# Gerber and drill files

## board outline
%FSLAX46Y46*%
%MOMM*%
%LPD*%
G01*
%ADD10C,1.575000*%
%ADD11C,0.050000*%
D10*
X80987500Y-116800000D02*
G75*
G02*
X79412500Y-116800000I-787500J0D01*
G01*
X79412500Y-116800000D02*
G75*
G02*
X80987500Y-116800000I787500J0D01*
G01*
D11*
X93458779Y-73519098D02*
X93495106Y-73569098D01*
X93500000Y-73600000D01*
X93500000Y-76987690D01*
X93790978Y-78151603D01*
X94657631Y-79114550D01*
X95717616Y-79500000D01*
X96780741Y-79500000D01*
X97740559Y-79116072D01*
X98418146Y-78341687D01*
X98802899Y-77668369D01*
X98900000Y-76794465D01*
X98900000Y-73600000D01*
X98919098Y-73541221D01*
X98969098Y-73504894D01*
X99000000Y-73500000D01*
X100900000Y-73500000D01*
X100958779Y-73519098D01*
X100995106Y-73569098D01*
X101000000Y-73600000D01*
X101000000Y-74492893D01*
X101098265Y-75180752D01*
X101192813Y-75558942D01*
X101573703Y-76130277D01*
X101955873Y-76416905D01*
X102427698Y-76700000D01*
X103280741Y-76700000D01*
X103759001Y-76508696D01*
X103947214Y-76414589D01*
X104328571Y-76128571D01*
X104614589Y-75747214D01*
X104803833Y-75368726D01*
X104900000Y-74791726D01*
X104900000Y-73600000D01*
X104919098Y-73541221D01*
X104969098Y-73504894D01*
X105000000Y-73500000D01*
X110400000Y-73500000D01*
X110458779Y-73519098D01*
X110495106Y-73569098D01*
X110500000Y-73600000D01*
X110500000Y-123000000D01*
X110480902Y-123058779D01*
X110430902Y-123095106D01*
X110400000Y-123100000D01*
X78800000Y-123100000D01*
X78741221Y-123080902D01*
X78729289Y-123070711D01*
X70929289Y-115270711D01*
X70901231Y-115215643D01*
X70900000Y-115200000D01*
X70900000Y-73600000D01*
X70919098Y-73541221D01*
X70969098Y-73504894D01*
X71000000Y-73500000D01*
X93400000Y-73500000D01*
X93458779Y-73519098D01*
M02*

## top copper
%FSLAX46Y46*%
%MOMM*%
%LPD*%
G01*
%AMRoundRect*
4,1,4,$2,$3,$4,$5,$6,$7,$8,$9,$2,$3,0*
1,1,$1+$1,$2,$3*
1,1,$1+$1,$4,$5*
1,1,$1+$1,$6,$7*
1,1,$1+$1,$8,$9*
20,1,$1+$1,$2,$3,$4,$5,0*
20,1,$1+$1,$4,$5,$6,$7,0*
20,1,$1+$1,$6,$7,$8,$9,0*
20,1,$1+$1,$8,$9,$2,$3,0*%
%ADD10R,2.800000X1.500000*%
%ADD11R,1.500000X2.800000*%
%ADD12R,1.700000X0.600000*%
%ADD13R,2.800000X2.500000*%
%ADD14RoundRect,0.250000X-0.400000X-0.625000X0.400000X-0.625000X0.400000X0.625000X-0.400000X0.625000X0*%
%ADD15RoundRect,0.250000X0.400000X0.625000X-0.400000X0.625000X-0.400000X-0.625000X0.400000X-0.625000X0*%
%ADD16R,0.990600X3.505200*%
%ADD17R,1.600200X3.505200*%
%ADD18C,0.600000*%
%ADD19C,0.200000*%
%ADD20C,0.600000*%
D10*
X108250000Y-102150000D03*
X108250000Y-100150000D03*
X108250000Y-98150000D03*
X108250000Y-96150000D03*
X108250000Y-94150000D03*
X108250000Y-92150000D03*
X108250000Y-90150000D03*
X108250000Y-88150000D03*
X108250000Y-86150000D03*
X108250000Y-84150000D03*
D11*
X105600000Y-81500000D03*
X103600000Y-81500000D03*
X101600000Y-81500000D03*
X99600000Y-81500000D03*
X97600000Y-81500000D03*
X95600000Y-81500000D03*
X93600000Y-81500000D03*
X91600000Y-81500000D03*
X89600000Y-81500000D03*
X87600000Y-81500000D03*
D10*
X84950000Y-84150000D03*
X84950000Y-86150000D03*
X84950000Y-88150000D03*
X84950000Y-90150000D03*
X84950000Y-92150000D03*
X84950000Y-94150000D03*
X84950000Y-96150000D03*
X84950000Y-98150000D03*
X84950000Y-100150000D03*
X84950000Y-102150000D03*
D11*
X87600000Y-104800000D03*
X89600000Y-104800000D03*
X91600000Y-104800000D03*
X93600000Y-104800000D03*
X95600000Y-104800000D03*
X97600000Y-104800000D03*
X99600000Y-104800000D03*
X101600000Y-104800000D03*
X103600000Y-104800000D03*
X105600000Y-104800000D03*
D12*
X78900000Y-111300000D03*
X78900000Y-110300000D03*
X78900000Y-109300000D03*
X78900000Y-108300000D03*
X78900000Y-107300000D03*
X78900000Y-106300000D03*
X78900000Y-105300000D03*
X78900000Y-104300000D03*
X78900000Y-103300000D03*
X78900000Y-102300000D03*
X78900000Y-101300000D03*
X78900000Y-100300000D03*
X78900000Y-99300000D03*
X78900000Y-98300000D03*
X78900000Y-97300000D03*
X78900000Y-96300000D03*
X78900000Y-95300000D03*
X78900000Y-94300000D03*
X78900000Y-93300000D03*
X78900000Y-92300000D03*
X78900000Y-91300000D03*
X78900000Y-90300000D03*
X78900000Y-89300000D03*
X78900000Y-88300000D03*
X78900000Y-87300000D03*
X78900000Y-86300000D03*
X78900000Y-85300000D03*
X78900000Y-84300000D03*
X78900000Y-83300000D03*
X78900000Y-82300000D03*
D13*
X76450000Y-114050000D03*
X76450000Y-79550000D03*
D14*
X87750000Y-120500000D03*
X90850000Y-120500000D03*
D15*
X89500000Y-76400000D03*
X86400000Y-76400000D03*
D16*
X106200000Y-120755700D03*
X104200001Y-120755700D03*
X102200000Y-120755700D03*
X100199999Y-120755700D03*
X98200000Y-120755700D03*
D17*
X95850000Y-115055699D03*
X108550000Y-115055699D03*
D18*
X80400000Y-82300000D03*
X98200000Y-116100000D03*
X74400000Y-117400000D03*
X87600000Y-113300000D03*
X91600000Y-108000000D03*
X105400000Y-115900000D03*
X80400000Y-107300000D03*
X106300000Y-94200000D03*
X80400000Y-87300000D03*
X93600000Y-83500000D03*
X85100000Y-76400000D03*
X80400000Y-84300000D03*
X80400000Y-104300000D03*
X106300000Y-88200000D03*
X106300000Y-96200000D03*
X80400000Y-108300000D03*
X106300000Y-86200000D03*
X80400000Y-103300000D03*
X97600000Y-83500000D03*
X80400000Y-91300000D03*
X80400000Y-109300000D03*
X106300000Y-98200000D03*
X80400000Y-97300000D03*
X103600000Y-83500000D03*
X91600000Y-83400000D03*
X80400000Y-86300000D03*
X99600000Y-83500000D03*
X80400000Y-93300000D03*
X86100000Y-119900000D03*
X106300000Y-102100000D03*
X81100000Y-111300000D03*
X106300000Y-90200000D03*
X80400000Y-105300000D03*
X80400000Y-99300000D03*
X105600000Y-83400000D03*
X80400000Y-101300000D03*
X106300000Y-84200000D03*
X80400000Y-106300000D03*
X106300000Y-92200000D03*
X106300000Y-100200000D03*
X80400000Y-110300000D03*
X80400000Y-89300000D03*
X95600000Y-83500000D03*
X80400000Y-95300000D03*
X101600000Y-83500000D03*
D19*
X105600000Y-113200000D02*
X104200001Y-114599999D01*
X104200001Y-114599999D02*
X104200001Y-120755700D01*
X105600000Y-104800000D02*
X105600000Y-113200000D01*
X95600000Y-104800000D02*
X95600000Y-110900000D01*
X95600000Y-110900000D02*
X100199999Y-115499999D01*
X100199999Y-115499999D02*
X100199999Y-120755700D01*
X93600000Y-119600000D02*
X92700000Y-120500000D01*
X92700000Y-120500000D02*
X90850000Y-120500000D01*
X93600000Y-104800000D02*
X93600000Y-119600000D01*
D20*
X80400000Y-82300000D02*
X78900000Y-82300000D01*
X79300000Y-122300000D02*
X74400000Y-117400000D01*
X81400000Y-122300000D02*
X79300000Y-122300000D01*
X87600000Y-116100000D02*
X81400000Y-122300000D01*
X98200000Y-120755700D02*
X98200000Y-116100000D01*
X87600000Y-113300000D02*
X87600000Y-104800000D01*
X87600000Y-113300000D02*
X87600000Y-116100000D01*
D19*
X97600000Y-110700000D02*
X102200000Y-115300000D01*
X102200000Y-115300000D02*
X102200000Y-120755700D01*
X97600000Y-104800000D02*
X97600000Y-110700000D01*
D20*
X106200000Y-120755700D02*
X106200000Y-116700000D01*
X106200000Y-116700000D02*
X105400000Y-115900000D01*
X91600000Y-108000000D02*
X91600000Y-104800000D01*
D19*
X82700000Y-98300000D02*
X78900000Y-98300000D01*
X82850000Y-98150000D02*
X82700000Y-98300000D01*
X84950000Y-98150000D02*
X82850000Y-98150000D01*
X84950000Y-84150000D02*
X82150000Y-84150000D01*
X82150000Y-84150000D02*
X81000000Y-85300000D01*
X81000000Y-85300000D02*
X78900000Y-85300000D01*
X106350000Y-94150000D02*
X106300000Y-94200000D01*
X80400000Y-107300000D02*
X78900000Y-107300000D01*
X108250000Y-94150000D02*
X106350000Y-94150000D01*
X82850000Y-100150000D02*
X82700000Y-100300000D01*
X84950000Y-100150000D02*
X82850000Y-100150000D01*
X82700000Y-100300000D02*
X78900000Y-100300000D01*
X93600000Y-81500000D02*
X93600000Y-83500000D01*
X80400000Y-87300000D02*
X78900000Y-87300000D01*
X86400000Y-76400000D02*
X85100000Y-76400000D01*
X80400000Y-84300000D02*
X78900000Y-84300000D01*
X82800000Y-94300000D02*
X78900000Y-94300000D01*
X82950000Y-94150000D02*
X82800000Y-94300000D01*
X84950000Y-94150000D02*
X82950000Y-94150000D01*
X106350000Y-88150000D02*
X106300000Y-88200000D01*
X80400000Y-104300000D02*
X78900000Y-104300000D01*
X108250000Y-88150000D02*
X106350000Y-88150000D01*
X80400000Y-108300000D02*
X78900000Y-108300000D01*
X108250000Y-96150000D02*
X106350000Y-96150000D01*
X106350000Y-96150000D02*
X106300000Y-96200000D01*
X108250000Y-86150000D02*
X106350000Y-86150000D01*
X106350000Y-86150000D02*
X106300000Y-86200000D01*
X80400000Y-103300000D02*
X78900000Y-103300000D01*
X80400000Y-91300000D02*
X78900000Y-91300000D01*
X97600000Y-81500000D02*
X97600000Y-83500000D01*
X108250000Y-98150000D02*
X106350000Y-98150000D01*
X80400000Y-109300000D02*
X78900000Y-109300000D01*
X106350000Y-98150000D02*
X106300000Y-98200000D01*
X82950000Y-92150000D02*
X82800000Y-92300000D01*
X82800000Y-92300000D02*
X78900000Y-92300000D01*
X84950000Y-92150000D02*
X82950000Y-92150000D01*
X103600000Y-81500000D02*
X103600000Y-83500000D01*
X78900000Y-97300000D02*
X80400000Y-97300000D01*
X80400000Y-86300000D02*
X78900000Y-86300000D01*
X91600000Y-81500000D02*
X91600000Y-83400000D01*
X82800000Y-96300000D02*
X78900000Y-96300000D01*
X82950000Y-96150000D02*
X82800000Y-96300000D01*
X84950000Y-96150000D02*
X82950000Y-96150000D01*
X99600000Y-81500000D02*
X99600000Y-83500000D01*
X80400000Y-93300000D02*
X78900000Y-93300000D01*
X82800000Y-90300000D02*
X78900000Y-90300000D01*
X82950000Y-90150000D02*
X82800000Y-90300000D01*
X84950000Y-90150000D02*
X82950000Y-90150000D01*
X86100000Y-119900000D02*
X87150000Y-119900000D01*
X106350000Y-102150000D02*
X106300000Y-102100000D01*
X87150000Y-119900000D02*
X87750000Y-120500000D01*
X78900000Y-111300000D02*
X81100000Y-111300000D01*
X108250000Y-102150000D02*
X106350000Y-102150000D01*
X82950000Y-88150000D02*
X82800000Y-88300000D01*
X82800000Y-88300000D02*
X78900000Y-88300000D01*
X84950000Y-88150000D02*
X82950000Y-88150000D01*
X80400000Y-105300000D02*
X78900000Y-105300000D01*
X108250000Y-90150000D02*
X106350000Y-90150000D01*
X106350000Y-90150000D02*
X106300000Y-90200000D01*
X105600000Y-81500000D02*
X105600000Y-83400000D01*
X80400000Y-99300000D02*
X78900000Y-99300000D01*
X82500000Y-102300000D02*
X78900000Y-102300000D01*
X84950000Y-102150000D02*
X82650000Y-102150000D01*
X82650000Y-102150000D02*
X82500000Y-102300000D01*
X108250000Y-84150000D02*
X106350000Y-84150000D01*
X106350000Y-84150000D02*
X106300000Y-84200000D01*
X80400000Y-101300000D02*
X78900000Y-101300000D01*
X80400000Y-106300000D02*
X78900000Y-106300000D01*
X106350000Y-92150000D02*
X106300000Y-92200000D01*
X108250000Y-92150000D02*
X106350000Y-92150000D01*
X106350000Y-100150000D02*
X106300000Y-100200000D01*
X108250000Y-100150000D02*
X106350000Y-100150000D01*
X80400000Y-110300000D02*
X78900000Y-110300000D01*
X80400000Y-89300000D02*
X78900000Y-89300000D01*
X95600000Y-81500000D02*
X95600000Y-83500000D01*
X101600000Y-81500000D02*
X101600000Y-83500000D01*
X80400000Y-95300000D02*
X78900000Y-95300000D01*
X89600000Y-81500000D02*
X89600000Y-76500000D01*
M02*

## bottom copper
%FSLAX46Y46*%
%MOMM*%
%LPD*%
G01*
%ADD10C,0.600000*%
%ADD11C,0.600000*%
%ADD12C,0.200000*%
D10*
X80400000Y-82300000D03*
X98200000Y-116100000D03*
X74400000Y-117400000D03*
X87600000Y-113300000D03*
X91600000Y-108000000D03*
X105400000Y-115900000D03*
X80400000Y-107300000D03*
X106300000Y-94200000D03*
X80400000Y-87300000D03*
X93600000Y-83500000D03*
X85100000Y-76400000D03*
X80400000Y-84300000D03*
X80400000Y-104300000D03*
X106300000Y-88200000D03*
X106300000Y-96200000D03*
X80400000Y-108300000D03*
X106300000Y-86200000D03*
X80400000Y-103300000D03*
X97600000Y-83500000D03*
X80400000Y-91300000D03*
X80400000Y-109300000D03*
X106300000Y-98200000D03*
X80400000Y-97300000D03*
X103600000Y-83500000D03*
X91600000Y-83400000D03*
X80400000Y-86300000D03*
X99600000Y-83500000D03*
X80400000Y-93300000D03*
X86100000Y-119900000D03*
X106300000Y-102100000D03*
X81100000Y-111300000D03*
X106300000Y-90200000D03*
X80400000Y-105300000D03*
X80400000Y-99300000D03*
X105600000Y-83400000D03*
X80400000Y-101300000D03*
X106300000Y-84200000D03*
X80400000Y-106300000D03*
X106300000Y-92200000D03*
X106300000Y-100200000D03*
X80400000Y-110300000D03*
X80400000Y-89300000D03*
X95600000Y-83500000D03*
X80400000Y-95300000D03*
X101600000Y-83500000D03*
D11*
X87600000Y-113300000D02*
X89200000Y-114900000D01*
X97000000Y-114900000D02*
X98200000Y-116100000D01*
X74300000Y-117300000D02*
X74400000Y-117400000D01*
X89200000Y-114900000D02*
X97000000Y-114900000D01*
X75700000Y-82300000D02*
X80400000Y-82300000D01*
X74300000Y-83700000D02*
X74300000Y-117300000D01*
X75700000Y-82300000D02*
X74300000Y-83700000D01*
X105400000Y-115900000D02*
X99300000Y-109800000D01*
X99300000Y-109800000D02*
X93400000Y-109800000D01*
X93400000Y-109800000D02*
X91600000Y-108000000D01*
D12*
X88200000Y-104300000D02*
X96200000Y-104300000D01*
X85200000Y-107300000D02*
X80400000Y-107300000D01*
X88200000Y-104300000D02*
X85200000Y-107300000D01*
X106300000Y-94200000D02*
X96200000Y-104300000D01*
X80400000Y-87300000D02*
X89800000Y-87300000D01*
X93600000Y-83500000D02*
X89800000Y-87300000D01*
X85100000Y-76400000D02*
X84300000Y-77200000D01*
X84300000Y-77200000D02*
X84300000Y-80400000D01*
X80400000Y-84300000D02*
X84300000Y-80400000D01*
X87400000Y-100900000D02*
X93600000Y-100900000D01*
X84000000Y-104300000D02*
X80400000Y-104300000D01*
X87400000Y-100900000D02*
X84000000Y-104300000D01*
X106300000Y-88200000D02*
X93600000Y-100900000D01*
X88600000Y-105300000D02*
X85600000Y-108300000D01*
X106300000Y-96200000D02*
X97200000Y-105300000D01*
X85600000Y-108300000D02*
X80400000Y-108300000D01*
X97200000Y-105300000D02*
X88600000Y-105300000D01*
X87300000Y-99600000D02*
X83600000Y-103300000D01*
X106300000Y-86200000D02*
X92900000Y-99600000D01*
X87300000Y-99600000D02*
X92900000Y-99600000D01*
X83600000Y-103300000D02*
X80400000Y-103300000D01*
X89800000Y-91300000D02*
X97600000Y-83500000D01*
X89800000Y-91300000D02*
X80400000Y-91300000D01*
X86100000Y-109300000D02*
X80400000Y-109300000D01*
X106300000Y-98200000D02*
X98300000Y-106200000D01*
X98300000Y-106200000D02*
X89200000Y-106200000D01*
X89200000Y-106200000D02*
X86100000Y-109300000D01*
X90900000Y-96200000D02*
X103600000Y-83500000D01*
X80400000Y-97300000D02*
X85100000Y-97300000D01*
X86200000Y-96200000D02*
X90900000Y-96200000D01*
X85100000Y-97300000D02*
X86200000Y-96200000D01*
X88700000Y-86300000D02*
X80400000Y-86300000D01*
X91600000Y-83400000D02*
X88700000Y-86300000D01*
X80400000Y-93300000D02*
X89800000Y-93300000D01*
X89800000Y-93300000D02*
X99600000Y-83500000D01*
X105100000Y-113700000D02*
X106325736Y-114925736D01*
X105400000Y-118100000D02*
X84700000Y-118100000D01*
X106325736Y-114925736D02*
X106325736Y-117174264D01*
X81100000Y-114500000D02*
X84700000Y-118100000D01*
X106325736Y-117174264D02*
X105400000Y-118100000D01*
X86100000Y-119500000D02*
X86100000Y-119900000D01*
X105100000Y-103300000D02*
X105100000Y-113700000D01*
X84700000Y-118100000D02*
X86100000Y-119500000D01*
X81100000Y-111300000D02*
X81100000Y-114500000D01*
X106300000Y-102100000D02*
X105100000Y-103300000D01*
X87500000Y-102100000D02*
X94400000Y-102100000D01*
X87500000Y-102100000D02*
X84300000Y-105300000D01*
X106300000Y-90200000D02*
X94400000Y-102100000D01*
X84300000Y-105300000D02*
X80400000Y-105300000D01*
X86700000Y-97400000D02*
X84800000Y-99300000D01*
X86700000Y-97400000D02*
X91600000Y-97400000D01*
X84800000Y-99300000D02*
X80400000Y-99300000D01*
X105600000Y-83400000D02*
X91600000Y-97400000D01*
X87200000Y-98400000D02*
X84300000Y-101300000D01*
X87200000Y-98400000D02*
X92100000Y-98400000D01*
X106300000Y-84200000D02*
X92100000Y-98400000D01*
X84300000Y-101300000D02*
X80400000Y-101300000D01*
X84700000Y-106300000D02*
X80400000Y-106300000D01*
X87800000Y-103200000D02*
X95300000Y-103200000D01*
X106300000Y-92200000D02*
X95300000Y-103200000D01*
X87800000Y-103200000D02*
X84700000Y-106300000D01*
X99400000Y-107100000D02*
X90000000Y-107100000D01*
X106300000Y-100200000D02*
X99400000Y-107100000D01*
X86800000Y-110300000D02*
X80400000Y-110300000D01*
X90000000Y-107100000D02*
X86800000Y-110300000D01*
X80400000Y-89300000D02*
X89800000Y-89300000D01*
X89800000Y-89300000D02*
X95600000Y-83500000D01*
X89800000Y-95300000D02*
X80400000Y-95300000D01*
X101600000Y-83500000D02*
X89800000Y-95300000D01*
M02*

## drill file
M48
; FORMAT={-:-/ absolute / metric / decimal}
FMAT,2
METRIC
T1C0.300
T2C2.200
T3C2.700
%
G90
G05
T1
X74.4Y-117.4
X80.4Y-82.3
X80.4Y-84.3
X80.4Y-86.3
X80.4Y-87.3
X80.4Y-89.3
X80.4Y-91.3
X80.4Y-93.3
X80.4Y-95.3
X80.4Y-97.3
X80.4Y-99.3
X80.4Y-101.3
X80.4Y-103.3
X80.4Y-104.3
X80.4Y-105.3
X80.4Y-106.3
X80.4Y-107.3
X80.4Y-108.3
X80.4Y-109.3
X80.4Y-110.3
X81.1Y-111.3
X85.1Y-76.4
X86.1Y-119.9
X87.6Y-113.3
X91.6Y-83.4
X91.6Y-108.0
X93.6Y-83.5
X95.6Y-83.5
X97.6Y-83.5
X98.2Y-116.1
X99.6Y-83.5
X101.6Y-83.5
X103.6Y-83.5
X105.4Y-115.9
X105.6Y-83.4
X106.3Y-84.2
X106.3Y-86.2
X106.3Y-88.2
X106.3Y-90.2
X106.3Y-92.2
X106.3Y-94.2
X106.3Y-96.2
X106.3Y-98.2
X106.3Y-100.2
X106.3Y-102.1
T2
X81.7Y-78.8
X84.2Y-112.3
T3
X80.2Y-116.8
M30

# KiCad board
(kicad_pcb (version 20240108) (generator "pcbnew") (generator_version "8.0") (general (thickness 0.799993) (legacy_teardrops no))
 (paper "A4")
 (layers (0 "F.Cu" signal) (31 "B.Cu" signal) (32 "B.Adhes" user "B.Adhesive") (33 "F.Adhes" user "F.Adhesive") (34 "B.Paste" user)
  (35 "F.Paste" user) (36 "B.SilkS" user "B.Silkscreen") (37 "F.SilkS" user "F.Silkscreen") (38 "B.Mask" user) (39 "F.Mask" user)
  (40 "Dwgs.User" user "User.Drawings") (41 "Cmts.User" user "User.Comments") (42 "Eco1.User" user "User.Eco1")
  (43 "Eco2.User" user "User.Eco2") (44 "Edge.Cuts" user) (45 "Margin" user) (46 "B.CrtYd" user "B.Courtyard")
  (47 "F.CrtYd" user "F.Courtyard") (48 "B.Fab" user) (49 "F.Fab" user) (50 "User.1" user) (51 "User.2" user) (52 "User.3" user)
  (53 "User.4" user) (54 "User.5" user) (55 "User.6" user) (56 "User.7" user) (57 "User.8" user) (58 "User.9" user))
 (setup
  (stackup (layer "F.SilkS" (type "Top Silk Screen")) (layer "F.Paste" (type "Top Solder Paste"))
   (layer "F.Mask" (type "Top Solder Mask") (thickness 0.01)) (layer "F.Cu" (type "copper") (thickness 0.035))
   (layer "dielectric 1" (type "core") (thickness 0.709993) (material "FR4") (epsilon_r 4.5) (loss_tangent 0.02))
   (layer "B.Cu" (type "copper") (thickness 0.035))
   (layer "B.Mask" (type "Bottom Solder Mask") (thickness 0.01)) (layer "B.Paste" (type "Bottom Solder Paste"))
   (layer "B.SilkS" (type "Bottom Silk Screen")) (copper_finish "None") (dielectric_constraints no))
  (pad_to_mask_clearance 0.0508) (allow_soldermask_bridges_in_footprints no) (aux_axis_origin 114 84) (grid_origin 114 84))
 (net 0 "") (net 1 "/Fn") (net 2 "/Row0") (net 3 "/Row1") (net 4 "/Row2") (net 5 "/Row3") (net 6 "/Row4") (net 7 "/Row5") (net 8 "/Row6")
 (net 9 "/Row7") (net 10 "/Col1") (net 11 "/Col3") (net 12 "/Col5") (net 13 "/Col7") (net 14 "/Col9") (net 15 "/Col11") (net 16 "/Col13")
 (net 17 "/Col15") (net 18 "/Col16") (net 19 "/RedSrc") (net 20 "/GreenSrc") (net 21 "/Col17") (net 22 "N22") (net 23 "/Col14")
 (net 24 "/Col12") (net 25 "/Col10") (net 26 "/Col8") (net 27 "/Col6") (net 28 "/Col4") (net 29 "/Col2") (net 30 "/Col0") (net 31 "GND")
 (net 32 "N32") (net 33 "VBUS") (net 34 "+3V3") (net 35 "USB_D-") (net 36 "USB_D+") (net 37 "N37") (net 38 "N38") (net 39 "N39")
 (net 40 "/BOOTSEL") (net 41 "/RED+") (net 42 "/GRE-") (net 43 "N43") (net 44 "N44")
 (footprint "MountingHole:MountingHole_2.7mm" (layer "F.Cu") (at 80.2 116.8)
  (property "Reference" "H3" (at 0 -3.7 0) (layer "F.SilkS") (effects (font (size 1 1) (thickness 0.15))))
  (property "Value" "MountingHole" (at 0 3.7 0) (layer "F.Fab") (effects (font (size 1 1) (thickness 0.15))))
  (pad "" np_thru_hole circle (at 0 0) (size 2.7 2.7) (drill 2.7) (layers "*.Cu" "*.Mask")))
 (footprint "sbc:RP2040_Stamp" (layer "F.Cu") (at 96.6 93.15 180)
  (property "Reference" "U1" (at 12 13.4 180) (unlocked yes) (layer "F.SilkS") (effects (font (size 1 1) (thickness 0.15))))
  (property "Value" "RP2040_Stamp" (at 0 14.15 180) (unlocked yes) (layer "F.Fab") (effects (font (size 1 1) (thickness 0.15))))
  (pad "1" smd rect (at -11.65 -9 180) (size 2.8 1.5) (layers "F.Cu" "F.Paste" "F.Mask") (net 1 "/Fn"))
  (pad "2" smd rect (at -11.65 -7 180) (size 2.8 1.5) (layers "F.Cu" "F.Paste" "F.Mask") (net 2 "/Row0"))
  (pad "3" smd rect (at -11.65 -5 180) (size 2.8 1.5) (layers "F.Cu" "F.Paste" "F.Mask") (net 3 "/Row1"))
  (pad "4" smd rect (at -11.65 -3 180) (size 2.8 1.5) (layers "F.Cu" "F.Paste" "F.Mask") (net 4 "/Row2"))
  (pad "5" smd rect (at -11.65 -1 180) (size 2.8 1.5) (layers "F.Cu" "F.Paste" "F.Mask") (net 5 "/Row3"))
  (pad "6" smd rect (at -11.65 1 180) (size 2.8 1.5) (layers "F.Cu" "F.Paste" "F.Mask") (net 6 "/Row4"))
  (pad "7" smd rect (at -11.65 3 180) (size 2.8 1.5) (layers "F.Cu" "F.Paste" "F.Mask") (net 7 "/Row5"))
  (pad "8" smd rect (at -11.65 5 180) (size 2.8 1.5) (layers "F.Cu" "F.Paste" "F.Mask") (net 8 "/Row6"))
  (pad "9" smd rect (at -11.65 7 180) (size 2.8 1.5) (layers "F.Cu" "F.Paste" "F.Mask") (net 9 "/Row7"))
  (pad "10" smd rect (at -11.65 9 180) (size 2.8 1.5) (layers "F.Cu" "F.Paste" "F.Mask") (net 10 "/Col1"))
  (pad "11" smd rect (at -9 11.65 90) (size 2.8 1.5) (layers "F.Cu" "F.Paste" "F.Mask") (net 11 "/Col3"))
  (pad "12" smd rect (at -7 11.65 90) (size 2.8 1.5) (layers "F.Cu" "F.Paste" "F.Mask") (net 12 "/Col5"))
  (pad "13" smd rect (at -5 11.65 90) (size 2.8 1.5) (layers "F.Cu" "F.Paste" "F.Mask") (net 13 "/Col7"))
  (pad "14" smd rect (at -3 11.65 90) (size 2.8 1.5) (layers "F.Cu" "F.Paste" "F.Mask") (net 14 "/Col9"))
  (pad "15" smd rect (at -1 11.65 90) (size 2.8 1.5) (layers "F.Cu" "F.Paste" "F.Mask") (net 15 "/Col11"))
  (pad "16" smd rect (at 1 11.65 90) (size 2.8 1.5) (layers "F.Cu" "F.Paste" "F.Mask") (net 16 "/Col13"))
  (pad "17" smd rect (at 3 11.65 90) (size 2.8 1.5) (layers "F.Cu" "F.Paste" "F.Mask") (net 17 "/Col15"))
  (pad "18" smd rect (at 5 11.65 90) (size 2.8 1.5) (layers "F.Cu" "F.Paste" "F.Mask") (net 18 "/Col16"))
  (pad "19" smd rect (at 7 11.65 90) (size 2.8 1.5) (layers "F.Cu" "F.Paste" "F.Mask") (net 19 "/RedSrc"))
  (pad "20" smd rect (at 9 11.65 90) (size 2.8 1.5) (layers "F.Cu" "F.Paste" "F.Mask") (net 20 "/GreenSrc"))
  (pad "21" smd rect (at 11.65 9 180) (size 2.8 1.5) (layers "F.Cu" "F.Paste" "F.Mask") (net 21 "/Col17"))
  (pad "22" smd rect (at 11.65 7 180) (size 2.8 1.5) (layers "F.Cu" "F.Paste" "F.Mask") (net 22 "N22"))
  (pad "23" smd rect (at 11.65 5 180) (size 2.8 1.5) (layers "F.Cu" "F.Paste" "F.Mask") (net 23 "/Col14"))
  (pad "24" smd rect (at 11.65 3 180) (size 2.8 1.5) (layers "F.Cu" "F.Paste" "F.Mask") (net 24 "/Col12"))
  (pad "25" smd rect (at 11.65 1 180) (size 2.8 1.5) (layers "F.Cu" "F.Paste" "F.Mask") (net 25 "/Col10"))
  (pad "26" smd rect (at 11.65 -1 180) (size 2.8 1.5) (layers "F.Cu" "F.Paste" "F.Mask") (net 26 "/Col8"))
  (pad "27" smd rect (at 11.65 -3 180) (size 2.8 1.5) (layers "F.Cu" "F.Paste" "F.Mask") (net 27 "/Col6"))
  (pad "28" smd rect (at 11.65 -5 180) (size 2.8 1.5) (layers "F.Cu" "F.Paste" "F.Mask") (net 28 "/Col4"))
  (pad "29" smd rect (at 11.65 -7 180) (size 2.8 1.5) (layers "F.Cu" "F.Paste" "F.Mask") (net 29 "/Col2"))
  (pad "30" smd rect (at 11.65 -9 180) (size 2.8 1.5) (layers "F.Cu" "F.Paste" "F.Mask") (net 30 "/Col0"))
  (pad "31" smd rect (at 9 -11.65 90) (size 2.8 1.5) (layers "F.Cu" "F.Paste" "F.Mask") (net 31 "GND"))
  (pad "32" smd rect (at 7 -11.65 90) (size 2.8 1.5) (layers "F.Cu" "F.Paste" "F.Mask") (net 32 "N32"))
  (pad "33" smd rect (at 5 -11.65 90) (size 2.8 1.5) (layers "F.Cu" "F.Paste" "F.Mask") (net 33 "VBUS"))
  (pad "34" smd rect (at 3 -11.65 90) (size 2.8 1.5) (layers "F.Cu" "F.Paste" "F.Mask") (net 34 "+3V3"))
  (pad "35" smd rect (at 1 -11.65 90) (size 2.8 1.5) (layers "F.Cu" "F.Paste" "F.Mask") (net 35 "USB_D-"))
  (pad "36" smd rect (at -1 -11.65 90) (size 2.8 1.5) (layers "F.Cu" "F.Paste" "F.Mask") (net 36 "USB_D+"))
  (pad "37" smd rect (at -3 -11.65 90) (size 2.8 1.5) (layers "F.Cu" "F.Paste" "F.Mask") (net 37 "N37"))
  (pad "38" smd rect (at -5 -11.65 90) (size 2.8 1.5) (layers "F.Cu" "F.Paste" "F.Mask") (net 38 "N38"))
  (pad "39" smd rect (at -7 -11.65 90) (size 2.8 1.5) (layers "F.Cu" "F.Paste" "F.Mask") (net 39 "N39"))
  (pad "40" smd rect (at -9 -11.65 90) (size 2.8 1.5) (layers "F.Cu" "F.Paste" "F.Mask") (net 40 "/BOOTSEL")))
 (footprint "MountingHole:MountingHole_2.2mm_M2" (layer "F.Cu") (at 81.7 78.8)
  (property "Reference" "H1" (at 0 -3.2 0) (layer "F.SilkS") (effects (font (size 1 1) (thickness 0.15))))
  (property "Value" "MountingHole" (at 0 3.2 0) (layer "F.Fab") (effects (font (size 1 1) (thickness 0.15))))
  (pad "" np_thru_hole circle (at 0 0) (size 2.2 2.2) (drill 2.2) (layers "*.Cu" "*.Mask")))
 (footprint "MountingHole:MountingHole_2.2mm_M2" (layer "F.Cu") (at 84.2 112.3)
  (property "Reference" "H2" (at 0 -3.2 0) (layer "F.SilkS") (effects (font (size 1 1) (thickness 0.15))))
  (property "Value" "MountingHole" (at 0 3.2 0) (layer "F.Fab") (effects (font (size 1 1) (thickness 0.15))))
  (pad "" np_thru_hole circle (at 0 0) (size 2.2 2.2) (drill 2.2) (layers "*.Cu" "*.Mask")))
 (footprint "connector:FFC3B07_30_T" (layer "F.Cu") (at 76.45 96.8 -90)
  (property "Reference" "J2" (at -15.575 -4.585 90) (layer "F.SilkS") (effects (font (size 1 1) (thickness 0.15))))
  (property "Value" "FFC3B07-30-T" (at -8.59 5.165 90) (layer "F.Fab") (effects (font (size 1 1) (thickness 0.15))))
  (pad "1" smd rect (at 14.5 -2.45 270) (size 0.6 1.7) (layers "F.Cu" "F.Paste" "F.Mask") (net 1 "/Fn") (solder_mask_margin 0.102))
  (pad "2" smd rect (at 13.5 -2.45 270) (size 0.6 1.7) (layers "F.Cu" "F.Paste" "F.Mask") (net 2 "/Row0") (solder_mask_margin 0.102))
  (pad "3" smd rect (at 12.5 -2.45 270) (size 0.6 1.7) (layers "F.Cu" "F.Paste" "F.Mask") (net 3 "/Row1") (solder_mask_margin 0.102))
  (pad "4" smd rect (at 11.5 -2.45 270) (size 0.6 1.7) (layers "F.Cu" "F.Paste" "F.Mask") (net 4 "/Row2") (solder_mask_margin 0.102))
  (pad "5" smd rect (at 10.5 -2.45 270) (size 0.6 1.7) (layers "F.Cu" "F.Paste" "F.Mask") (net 5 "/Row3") (solder_mask_margin 0.102))
  (pad "6" smd rect (at 9.5 -2.45 270) (size 0.6 1.7) (layers "F.Cu" "F.Paste" "F.Mask") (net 6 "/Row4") (solder_mask_margin 0.102))
  (pad "7" smd rect (at 8.5 -2.45 270) (size 0.6 1.7) (layers "F.Cu" "F.Paste" "F.Mask") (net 7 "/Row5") (solder_mask_margin 0.102))
  (pad "8" smd rect (at 7.5 -2.45 270) (size 0.6 1.7) (layers "F.Cu" "F.Paste" "F.Mask") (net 8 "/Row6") (solder_mask_margin 0.102))
  (pad "9" smd rect (at 6.5 -2.45 270) (size 0.6 1.7) (layers "F.Cu" "F.Paste" "F.Mask") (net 9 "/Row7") (solder_mask_margin 0.102))
  (pad "10" smd rect (at 5.5 -2.45 270) (size 0.6 1.7) (layers "F.Cu" "F.Paste" "F.Mask") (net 30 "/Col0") (solder_mask_margin 0.102))
  (pad "11" smd rect (at 4.5 -2.45 270) (size 0.6 1.7) (layers "F.Cu" "F.Paste" "F.Mask") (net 10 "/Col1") (solder_mask_margin 0.102))
  (pad "12" smd rect (at 3.5 -2.45 270) (size 0.6 1.7) (layers "F.Cu" "F.Paste" "F.Mask") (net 29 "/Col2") (solder_mask_margin 0.102))
  (pad "13" smd rect (at 2.5 -2.45 270) (size 0.6 1.7) (layers "F.Cu" "F.Paste" "F.Mask") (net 11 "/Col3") (solder_mask_margin 0.102))
  (pad "14" smd rect (at 1.5 -2.45 270) (size 0.6 1.7) (layers "F.Cu" "F.Paste" "F.Mask") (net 28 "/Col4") (solder_mask_margin 0.102))
  (pad "15" smd rect (at 0.5 -2.45 270) (size 0.6 1.7) (layers "F.Cu" "F.Paste" "F.Mask") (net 12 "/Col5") (solder_mask_margin 0.102))
  (pad "16" smd rect (at -0.5 -2.45 270) (size 0.6 1.7) (layers "F.Cu" "F.Paste" "F.Mask") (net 27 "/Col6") (solder_mask_margin 0.102))
  (pad "17" smd rect (at -1.5 -2.45 270) (size 0.6 1.7) (layers "F.Cu" "F.Paste" "F.Mask") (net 13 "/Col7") (solder_mask_margin 0.102))
  (pad "18" smd rect (at -2.5 -2.45 270) (size 0.6 1.7) (layers "F.Cu" "F.Paste" "F.Mask") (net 26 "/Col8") (solder_mask_margin 0.102))
  (pad "19" smd rect (at -3.5 -2.45 270) (size 0.6 1.7) (layers "F.Cu" "F.Paste" "F.Mask") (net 14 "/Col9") (solder_mask_margin 0.102))
  (pad "20" smd rect (at -4.5 -2.45 270) (size 0.6 1.7) (layers "F.Cu" "F.Paste" "F.Mask") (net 25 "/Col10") (solder_mask_margin 0.102))
  (pad "21" smd rect (at -5.5 -2.45 270) (size 0.6 1.7) (layers "F.Cu" "F.Paste" "F.Mask") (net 15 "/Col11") (solder_mask_margin 0.102))
  (pad "22" smd rect (at -6.5 -2.45 270) (size 0.6 1.7) (layers "F.Cu" "F.Paste" "F.Mask") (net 24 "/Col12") (solder_mask_margin 0.102))
  (pad "23" smd rect (at -7.5 -2.45 270) (size 0.6 1.7) (layers "F.Cu" "F.Paste" "F.Mask") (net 16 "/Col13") (solder_mask_margin 0.102))
  (pad "24" smd rect (at -8.5 -2.45 270) (size 0.6 1.7) (layers "F.Cu" "F.Paste" "F.Mask") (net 23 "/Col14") (solder_mask_margin 0.102))
  (pad "25" smd rect (at -9.5 -2.45 270) (size 0.6 1.7) (layers "F.Cu" "F.Paste" "F.Mask") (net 17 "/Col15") (solder_mask_margin 0.102))
  (pad "26" smd rect (at -10.5 -2.45 270) (size 0.6 1.7) (layers "F.Cu" "F.Paste" "F.Mask") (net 18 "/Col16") (solder_mask_margin 0.102))
  (pad "27" smd rect (at -11.5 -2.45 270) (size 0.6 1.7) (layers "F.Cu" "F.Paste" "F.Mask") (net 21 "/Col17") (solder_mask_margin 0.102))
  (pad "28" smd rect (at -12.5 -2.45 270) (size 0.6 1.7) (layers "F.Cu" "F.Paste" "F.Mask") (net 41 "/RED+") (solder_mask_margin 0.102))
  (pad "29" smd rect (at -13.5 -2.45 270) (size 0.6 1.7) (layers "F.Cu" "F.Paste" "F.Mask") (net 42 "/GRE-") (solder_mask_margin 0.102))
  (pad "30" smd rect (at -14.5 -2.45 270) (size 0.6 1.7) (layers "F.Cu" "F.Paste" "F.Mask") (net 31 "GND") (solder_mask_margin 0.102))
  (pad "S1" smd rect (at 17.25 0 270) (size 2.5 2.8) (layers "F.Cu" "F.Paste" "F.Mask") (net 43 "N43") (solder_mask_margin 0.102))
  (pad "S2" smd rect (at -17.25 0 270) (size 2.5 2.8) (layers "F.Cu" "F.Paste" "F.Mask") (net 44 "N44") (solder_mask_margin 0.102)))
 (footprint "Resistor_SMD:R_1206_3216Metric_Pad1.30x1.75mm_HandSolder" (layer "F.Cu") (at 89.3 120.5)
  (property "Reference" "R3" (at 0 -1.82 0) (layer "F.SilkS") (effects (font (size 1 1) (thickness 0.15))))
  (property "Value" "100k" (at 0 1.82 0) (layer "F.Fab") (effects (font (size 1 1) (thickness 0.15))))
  (pad "1" smd roundrect (at -1.55 0) (size 1.3 1.75) (layers "F.Cu" "F.Paste" "F.Mask") (roundrect_rratio 0.192308) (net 1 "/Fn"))
  (pad "2" smd roundrect (at 1.55 0) (size 1.3 1.75) (layers "F.Cu" "F.Paste" "F.Mask") (roundrect_rratio 0.192308) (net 34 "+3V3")))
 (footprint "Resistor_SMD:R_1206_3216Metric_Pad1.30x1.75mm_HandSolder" (layer "F.Cu") (at 87.95 76.4 180)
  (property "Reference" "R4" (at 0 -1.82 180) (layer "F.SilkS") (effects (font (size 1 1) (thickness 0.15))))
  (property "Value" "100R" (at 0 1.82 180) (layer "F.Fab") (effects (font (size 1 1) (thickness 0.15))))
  (pad "1" smd roundrect (at -1.55 0 180) (size 1.3 1.75) (layers "F.Cu" "F.Paste" "F.Mask") (roundrect_rratio 0.192308) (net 19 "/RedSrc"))
  (pad "2" smd roundrect (at 1.55 0 180) (size 1.3 1.75) (layers "F.Cu" "F.Paste" "F.Mask") (roundrect_rratio 0.192308) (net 41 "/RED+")))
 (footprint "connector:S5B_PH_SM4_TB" (layer "F.Cu") (at 102.2 117.3)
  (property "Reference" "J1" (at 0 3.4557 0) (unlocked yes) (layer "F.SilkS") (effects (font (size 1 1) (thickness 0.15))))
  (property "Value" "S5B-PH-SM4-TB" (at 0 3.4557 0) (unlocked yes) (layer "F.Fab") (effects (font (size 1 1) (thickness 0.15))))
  (pad "1" smd rect (at 4 3.4557) (size 0.9906 3.5052) (layers "F.Cu" "F.Paste" "F.Mask") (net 33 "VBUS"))
  (pad "2" smd rect (at 2.000001 3.4557) (size 0.9906 3.5052) (layers "F.Cu" "F.Paste" "F.Mask") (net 40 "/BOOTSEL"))
  (pad "3" smd rect (at 0 3.4557) (size 0.9906 3.5052) (layers "F.Cu" "F.Paste" "F.Mask") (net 36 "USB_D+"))
  (pad "4" smd rect (at -2.000001 3.4557) (size 0.9906 3.5052) (layers "F.Cu" "F.Paste" "F.Mask") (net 35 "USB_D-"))
  (pad "5" smd rect (at -4 3.4557) (size 0.9906 3.5052) (layers "F.Cu" "F.Paste" "F.Mask") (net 31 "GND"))
  (pad "6" smd rect (at -6.35 -2.244301) (size 1.6002 3.5052) (layers "F.Cu" "F.Paste" "F.Mask"))
  (pad "7" smd rect (at 6.35 -2.244301) (size 1.6002 3.5052) (layers "F.Cu" "F.Paste" "F.Mask")))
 (gr_circle (center 80.2 116.8) (end 81.75 116.8) (stroke (width 0.05) (type solid)) (fill solid) (layer "Edge.Cuts"))
 (gr_poly
  (pts (xy 93.458779 73.519098) (xy 93.495106 73.569098) (xy 93.5 73.6) (xy 93.5 76.98769) (xy 93.790978 78.151603) (xy 94.657631 79.11455)
   (xy 95.717616 79.5) (xy 96.780741 79.5) (xy 97.740559 79.116072) (xy 98.418146 78.341687) (xy 98.802899 77.668369) (xy 98.9 76.794465)
   (xy 98.9 73.6) (xy 98.919098 73.541221) (xy 98.969098 73.504894) (xy 99 73.5) (xy 100.9 73.5) (xy 100.958779 73.519098)
   (xy 100.995106 73.569098) (xy 101 73.6) (xy 101 74.492893) (xy 101.098265 75.180752) (xy 101.192813 75.558942) (xy 101.573703 76.130277)
   (xy 101.955873 76.416905) (xy 102.427698 76.7) (xy 103.280741 76.7) (xy 103.759001 76.508696) (xy 103.947214 76.414589)
   (xy 104.328571 76.128571) (xy 104.614589 75.747214) (xy 104.803833 75.368726) (xy 104.9 74.791726) (xy 104.9 73.6)
   (xy 104.919098 73.541221) (xy 104.969098 73.504894) (xy 105 73.5) (xy 110.4 73.5) (xy 110.458779 73.519098) (xy 110.495106 73.569098)
   (xy 110.5 73.6) (xy 110.5 123) (xy 110.480902 123.058779) (xy 110.430902 123.095106) (xy 110.4 123.1) (xy 78.8 123.1)
   (xy 78.741221 123.080902) (xy 78.729289 123.070711) (xy 70.929289 115.270711) (xy 70.901231 115.215643) (xy 70.9 115.2) (xy 70.9 73.6)
   (xy 70.919098 73.541221) (xy 70.969098 73.504894) (xy 71 73.5) (xy 93.4 73.5))
  (stroke (width 0.05) (type solid)) (fill none) (layer "Edge.Cuts"))
 (segment (start 105.6 113.2) (end 104.200001 114.599999) (width 0.2) (layer "F.Cu") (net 40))
 (segment (start 104.200001 114.599999) (end 104.200001 120.7557) (width 0.2) (layer "F.Cu") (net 40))
 (segment (start 105.6 104.8) (end 105.6 113.2) (width 0.2) (layer "F.Cu") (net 40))
 (segment (start 95.6 104.8) (end 95.6 110.9) (width 0.2) (layer "F.Cu") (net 35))
 (segment (start 95.6 110.9) (end 100.199999 115.499999) (width 0.2) (layer "F.Cu") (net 35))
 (segment (start 100.199999 115.499999) (end 100.199999 120.7557) (width 0.2) (layer "F.Cu") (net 35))
 (segment (start 93.6 119.6) (end 92.7 120.5) (width 0.2) (layer "F.Cu") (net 34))
 (segment (start 92.7 120.5) (end 90.85 120.5) (width 0.2) (layer "F.Cu") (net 34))
 (segment (start 93.6 104.8) (end 93.6 119.6) (width 0.2) (layer "F.Cu") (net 34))
 (segment (start 80.4 82.3) (end 78.9 82.3) (width 0.6) (layer "F.Cu") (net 31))
 (segment (start 79.3 122.3) (end 74.4 117.4) (width 0.6) (layer "F.Cu") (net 31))
 (segment (start 81.4 122.3) (end 79.3 122.3) (width 0.6) (layer "F.Cu") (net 31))
 (segment (start 87.6 116.1) (end 81.4 122.3) (width 0.6) (layer "F.Cu") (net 31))
 (segment (start 98.2 120.7557) (end 98.2 116.1) (width 0.6) (layer "F.Cu") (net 31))
 (segment (start 87.6 113.3) (end 87.6 104.8) (width 0.6) (layer "F.Cu") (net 31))
 (segment (start 87.6 113.3) (end 87.6 116.1) (width 0.6) (layer "F.Cu") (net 31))
 (via (at 80.4 82.3) (size 0.6) (drill 0.3) (layers "F.Cu" "B.Cu") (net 31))
 (via (at 98.2 116.1) (size 0.6) (drill 0.3) (layers "F.Cu" "B.Cu") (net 31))
 (via (at 74.4 117.4) (size 0.6) (drill 0.3) (layers "F.Cu" "B.Cu") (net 31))
 (via (at 87.6 113.3) (size 0.6) (drill 0.3) (layers "F.Cu" "B.Cu") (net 31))
 (segment (start 87.6 113.3) (end 89.2 114.9) (width 0.6) (layer "B.Cu") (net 31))
 (segment (start 97 114.9) (end 98.2 116.1) (width 0.6) (layer "B.Cu") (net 31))
 (segment (start 74.3 117.3) (end 74.4 117.4) (width 0.6) (layer "B.Cu") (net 31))
 (segment (start 89.2 114.9) (end 97 114.9) (width 0.6) (layer "B.Cu") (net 31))
 (segment (start 75.7 82.3) (end 80.4 82.3) (width 0.6) (layer "B.Cu") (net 31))
 (segment (start 74.3 83.7) (end 74.3 117.3) (width 0.6) (layer "B.Cu") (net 31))
 (segment (start 75.7 82.3) (end 74.3 83.7) (width 0.6) (layer "B.Cu") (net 31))
 (segment (start 97.6 110.7) (end 102.2 115.3) (width 0.2) (layer "F.Cu") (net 36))
 (segment (start 102.2 115.3) (end 102.2 120.7557) (width 0.2) (layer "F.Cu") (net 36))
 (segment (start 97.6 104.8) (end 97.6 110.7) (width 0.2) (layer "F.Cu") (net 36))
 (segment (start 106.2 120.7557) (end 106.2 116.7) (width 0.6) (layer "F.Cu") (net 33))
 (segment (start 106.2 116.7) (end 105.4 115.9) (width 0.6) (layer "F.Cu") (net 33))
 (segment (start 91.6 108) (end 91.6 104.8) (width 0.6) (layer "F.Cu") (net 33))
 (via (at 91.6 108) (size 0.6) (drill 0.3) (layers "F.Cu" "B.Cu") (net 33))
 (via (at 105.4 115.9) (size 0.6) (drill 0.3) (layers "F.Cu" "B.Cu") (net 33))
 (segment (start 105.4 115.9) (end 99.3 109.8) (width 0.6) (layer "B.Cu") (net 33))
 (segment (start 99.3 109.8) (end 93.4 109.8) (width 0.6) (layer "B.Cu") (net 33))
 (segment (start 93.4 109.8) (end 91.6 108) (width 0.6) (layer "B.Cu") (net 33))
 (segment (start 82.7 98.3) (end 78.9 98.3) (width 0.2) (layer "F.Cu") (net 28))
 (segment (start 82.85 98.15) (end 82.7 98.3) (width 0.2) (layer "F.Cu") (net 28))
 (segment (start 84.95 98.15) (end 82.85 98.15) (width 0.2) (layer "F.Cu") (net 28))
 (segment (start 84.95 84.15) (end 82.15 84.15) (width 0.2) (layer "F.Cu") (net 21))
 (segment (start 82.15 84.15) (end 81 85.3) (width 0.2) (layer "F.Cu") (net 21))
 (segment (start 81 85.3) (end 78.9 85.3) (width 0.2) (layer "F.Cu") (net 21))
 (segment (start 106.35 94.15) (end 106.3 94.2) (width 0.2) (layer "F.Cu") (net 5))
 (segment (start 80.4 107.3) (end 78.9 107.3) (width 0.2) (layer "F.Cu") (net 5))
 (segment (start 108.25 94.15) (end 106.35 94.15) (width 0.2) (layer "F.Cu") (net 5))
 (via (at 80.4 107.3) (size 0.6) (drill 0.3) (layers "F.Cu" "B.Cu") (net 5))
 (via (at 106.3 94.2) (size 0.6) (drill 0.3) (layers "F.Cu" "B.Cu") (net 5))
 (segment (start 88.2 104.3) (end 96.2 104.3) (width 0.2) (layer "B.Cu") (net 5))
 (segment (start 85.2 107.3) (end 80.4 107.3) (width 0.2) (layer "B.Cu") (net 5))
 (segment (start 88.2 104.3) (end 85.2 107.3) (width 0.2) (layer "B.Cu") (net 5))
 (segment (start 106.3 94.2) (end 96.2 104.3) (width 0.2) (layer "B.Cu") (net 5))
 (segment (start 82.85 100.15) (end 82.7 100.3) (width 0.2) (layer "F.Cu") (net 29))
 (segment (start 84.95 100.15) (end 82.85 100.15) (width 0.2) (layer "F.Cu") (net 29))
 (segment (start 82.7 100.3) (end 78.9 100.3) (width 0.2) (layer "F.Cu") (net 29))
 (segment (start 93.6 81.5) (end 93.6 83.5) (width 0.2) (layer "F.Cu") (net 17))
 (segment (start 80.4 87.3) (end 78.9 87.3) (width 0.2) (layer "F.Cu") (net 17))
 (via (at 80.4 87.3) (size 0.6) (drill 0.3) (layers "F.Cu" "B.Cu") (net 17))
 (via (at 93.6 83.5) (size 0.6) (drill 0.3) (layers "F.Cu" "B.Cu") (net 17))
 (segment (start 80.4 87.3) (end 89.8 87.3) (width 0.2) (layer "B.Cu") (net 17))
 (segment (start 93.6 83.5) (end 89.8 87.3) (width 0.2) (layer "B.Cu") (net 17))
 (segment (start 86.4 76.4) (end 85.1 76.4) (width 0.2) (layer "F.Cu") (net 41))
 (segment (start 80.4 84.3) (end 78.9 84.3) (width 0.2) (layer "F.Cu") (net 41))
 (via (at 85.1 76.4) (size 0.6) (drill 0.3) (layers "F.Cu" "B.Cu") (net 41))
 (via (at 80.4 84.3) (size 0.6) (drill 0.3) (layers "F.Cu" "B.Cu") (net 41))
 (segment (start 85.1 76.4) (end 84.3 77.2) (width 0.2) (layer "B.Cu") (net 41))
 (segment (start 84.3 77.2) (end 84.3 80.4) (width 0.2) (layer "B.Cu") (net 41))
 (segment (start 80.4 84.3) (end 84.3 80.4) (width 0.2) (layer "B.Cu") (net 41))
 (segment (start 82.8 94.3) (end 78.9 94.3) (width 0.2) (layer "F.Cu") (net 26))
 (segment (start 82.95 94.15) (end 82.8 94.3) (width 0.2) (layer "F.Cu") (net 26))
 (segment (start 84.95 94.15) (end 82.95 94.15) (width 0.2) (layer "F.Cu") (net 26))
 (segment (start 106.35 88.15) (end 106.3 88.2) (width 0.2) (layer "F.Cu") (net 8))
 (segment (start 80.4 104.3) (end 78.9 104.3) (width 0.2) (layer "F.Cu") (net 8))
 (segment (start 108.25 88.15) (end 106.35 88.15) (width 0.2) (layer "F.Cu") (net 8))
 (via (at 80.4 104.3) (size 0.6) (drill 0.3) (layers "F.Cu" "B.Cu") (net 8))
 (via (at 106.3 88.2) (size 0.6) (drill 0.3) (layers "F.Cu" "B.Cu") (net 8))
 (segment (start 87.4 100.9) (end 93.6 100.9) (width 0.2) (layer "B.Cu") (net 8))
 (segment (start 84 104.3) (end 80.4 104.3) (width 0.2) (layer "B.Cu") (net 8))
 (segment (start 87.4 100.9) (end 84 104.3) (width 0.2) (layer "B.Cu") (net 8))
 (segment (start 106.3 88.2) (end 93.6 100.9) (width 0.2) (layer "B.Cu") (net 8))
 (segment (start 80.4 108.3) (end 78.9 108.3) (width 0.2) (layer "F.Cu") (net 4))
 (segment (start 108.25 96.15) (end 106.35 96.15) (width 0.2) (layer "F.Cu") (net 4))
 (segment (start 106.35 96.15) (end 106.3 96.2) (width 0.2) (layer "F.Cu") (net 4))
 (via (at 106.3 96.2) (size 0.6) (drill 0.3) (layers "F.Cu" "B.Cu") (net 4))
 (via (at 80.4 108.3) (size 0.6) (drill 0.3) (layers "F.Cu" "B.Cu") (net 4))
 (segment (start 88.6 105.3) (end 85.6 108.3) (width 0.2) (layer "B.Cu") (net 4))
 (segment (start 106.3 96.2) (end 97.2 105.3) (width 0.2) (layer "B.Cu") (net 4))
 (segment (start 85.6 108.3) (end 80.4 108.3) (width 0.2) (layer "B.Cu") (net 4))
 (segment (start 97.2 105.3) (end 88.6 105.3) (width 0.2) (layer "B.Cu") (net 4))
 (segment (start 108.25 86.15) (end 106.35 86.15) (width 0.2) (layer "F.Cu") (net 9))
 (segment (start 106.35 86.15) (end 106.3 86.2) (width 0.2) (layer "F.Cu") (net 9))
 (segment (start 80.4 103.3) (end 78.9 103.3) (width 0.2) (layer "F.Cu") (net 9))
 (via (at 106.3 86.2) (size 0.6) (drill 0.3) (layers "F.Cu" "B.Cu") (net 9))
 (via (at 80.4 103.3) (size 0.6) (drill 0.3) (layers "F.Cu" "B.Cu") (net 9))
 (segment (start 87.3 99.6) (end 83.6 103.3) (width 0.2) (layer "B.Cu") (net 9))
 (segment (start 106.3 86.2) (end 92.9 99.6) (width 0.2) (layer "B.Cu") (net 9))
 (segment (start 87.3 99.6) (end 92.9 99.6) (width 0.2) (layer "B.Cu") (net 9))
 (segment (start 83.6 103.3) (end 80.4 103.3) (width 0.2) (layer "B.Cu") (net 9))
 (segment (start 80.4 91.3) (end 78.9 91.3) (width 0.2) (layer "F.Cu") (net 15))
 (segment (start 97.6 81.5) (end 97.6 83.5) (width 0.2) (layer "F.Cu") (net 15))
 (via (at 97.6 83.5) (size 0.6) (drill 0.3) (layers "F.Cu" "B.Cu") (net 15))
 (via (at 80.4 91.3) (size 0.6) (drill 0.3) (layers "F.Cu" "B.Cu") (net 15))
 (segment (start 89.8 91.3) (end 97.6 83.5) (width 0.2) (layer "B.Cu") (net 15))
 (segment (start 89.8 91.3) (end 80.4 91.3) (width 0.2) (layer "B.Cu") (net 15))
 (segment (start 108.25 98.15) (end 106.35 98.15) (width 0.2) (layer "F.Cu") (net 3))
 (segment (start 80.4 109.3) (end 78.9 109.3) (width 0.2) (layer "F.Cu") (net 3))
 (segment (start 106.35 98.15) (end 106.3 98.2) (width 0.2) (layer "F.Cu") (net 3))
 (via (at 80.4 109.3) (size 0.6) (drill 0.3) (layers "F.Cu" "B.Cu") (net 3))
 (via (at 106.3 98.2) (size 0.6) (drill 0.3) (layers "F.Cu" "B.Cu") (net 3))
 (segment (start 86.1 109.3) (end 80.4 109.3) (width 0.2) (layer "B.Cu") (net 3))
 (segment (start 106.3 98.2) (end 98.3 106.2) (width 0.2) (layer "B.Cu") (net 3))
 (segment (start 98.3 106.2) (end 89.2 106.2) (width 0.2) (layer "B.Cu") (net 3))
 (segment (start 89.2 106.2) (end 86.1 109.3) (width 0.2) (layer "B.Cu") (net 3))
 (segment (start 82.95 92.15) (end 82.8 92.3) (width 0.2) (layer "F.Cu") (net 25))
 (segment (start 82.8 92.3) (end 78.9 92.3) (width 0.2) (layer "F.Cu") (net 25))
 (segment (start 84.95 92.15) (end 82.95 92.15) (width 0.2) (layer "F.Cu") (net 25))
 (segment (start 103.6 81.5) (end 103.6 83.5) (width 0.2) (layer "F.Cu") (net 12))
 (segment (start 78.9 97.3) (end 80.4 97.3) (width 0.2) (layer "F.Cu") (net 12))
 (via (at 80.4 97.3) (size 0.6) (drill 0.3) (layers "F.Cu" "B.Cu") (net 12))
 (via (at 103.6 83.5) (size 0.6) (drill 0.3) (layers "F.Cu" "B.Cu") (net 12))
 (segment (start 90.9 96.2) (end 103.6 83.5) (width 0.2) (layer "B.Cu") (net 12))
 (segment (start 80.4 97.3) (end 85.1 97.3) (width 0.2) (layer "B.Cu") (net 12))
 (segment (start 86.2 96.2) (end 90.9 96.2) (width 0.2) (layer "B.Cu") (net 12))
 (segment (start 85.1 97.3) (end 86.2 96.2) (width 0.2) (layer "B.Cu") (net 12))
 (segment (start 80.4 86.3) (end 78.9 86.3) (width 0.2) (layer "F.Cu") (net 18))
 (segment (start 91.6 81.5) (end 91.6 83.4) (width 0.2) (layer "F.Cu") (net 18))
 (via (at 91.6 83.4) (size 0.6) (drill 0.3) (layers "F.Cu" "B.Cu") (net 18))
 (via (at 80.4 86.3) (size 0.6) (drill 0.3) (layers "F.Cu" "B.Cu") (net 18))
 (segment (start 88.7 86.3) (end 80.4 86.3) (width 0.2) (layer "B.Cu") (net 18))
 (segment (start 91.6 83.4) (end 88.7 86.3) (width 0.2) (layer "B.Cu") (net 18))
 (segment (start 82.8 96.3) (end 78.9 96.3) (width 0.2) (layer "F.Cu") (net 27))
 (segment (start 82.95 96.15) (end 82.8 96.3) (width 0.2) (layer "F.Cu") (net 27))
 (segment (start 84.95 96.15) (end 82.95 96.15) (width 0.2) (layer "F.Cu") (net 27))
 (segment (start 99.6 81.5) (end 99.6 83.5) (width 0.2) (layer "F.Cu") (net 14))
 (segment (start 80.4 93.3) (end 78.9 93.3) (width 0.2) (layer "F.Cu") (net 14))
 (via (at 99.6 83.5) (size 0.6) (drill 0.3) (layers "F.Cu" "B.Cu") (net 14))
 (via (at 80.4 93.3) (size 0.6) (drill 0.3) (layers "F.Cu" "B.Cu") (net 14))
 (segment (start 80.4 93.3) (end 89.8 93.3) (width 0.2) (layer "B.Cu") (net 14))
 (segment (start 89.8 93.3) (end 99.6 83.5) (width 0.2) (layer "B.Cu") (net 14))
 (segment (start 82.8 90.3) (end 78.9 90.3) (width 0.2) (layer "F.Cu") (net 24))
 (segment (start 82.95 90.15) (end 82.8 90.3) (width 0.2) (layer "F.Cu") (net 24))
 (segment (start 84.95 90.15) (end 82.95 90.15) (width 0.2) (layer "F.Cu") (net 24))
 (segment (start 86.1 119.9) (end 87.15 119.9) (width 0.2) (layer "F.Cu") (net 1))
 (segment (start 106.35 102.15) (end 106.3 102.1) (width 0.2) (layer "F.Cu") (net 1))
 (segment (start 87.15 119.9) (end 87.75 120.5) (width 0.2) (layer "F.Cu") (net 1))
 (segment (start 78.9 111.3) (end 81.1 111.3) (width 0.2) (layer "F.Cu") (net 1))
 (segment (start 108.25 102.15) (end 106.35 102.15) (width 0.2) (layer "F.Cu") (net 1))
 (via (at 86.1 119.9) (size 0.6) (drill 0.3) (layers "F.Cu" "B.Cu") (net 1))
 (via (at 106.3 102.1) (size 0.6) (drill 0.3) (layers "F.Cu" "B.Cu") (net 1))
 (via (at 81.1 111.3) (size 0.6) (drill 0.3) (layers "F.Cu" "B.Cu") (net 1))
 (segment (start 105.1 113.7) (end 106.325736 114.925736) (width 0.2) (layer "B.Cu") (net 1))
 (segment (start 105.4 118.1) (end 84.7 118.1) (width 0.2) (layer "B.Cu") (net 1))
 (segment (start 106.325736 114.925736) (end 106.325736 117.174264) (width 0.2) (layer "B.Cu") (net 1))
 (segment (start 81.1 114.5) (end 84.7 118.1) (width 0.2) (layer "B.Cu") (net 1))
 (segment (start 106.325736 117.174264) (end 105.4 118.1) (width 0.2) (layer "B.Cu") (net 1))
 (segment (start 86.1 119.5) (end 86.1 119.9) (width 0.2) (layer "B.Cu") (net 1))
 (segment (start 105.1 103.3) (end 105.1 113.7) (width 0.2) (layer "B.Cu") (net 1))
 (segment (start 84.7 118.1) (end 86.1 119.5) (width 0.2) (layer "B.Cu") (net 1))
 (segment (start 81.1 111.3) (end 81.1 114.5) (width 0.2) (layer "B.Cu") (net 1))
 (segment (start 106.3 102.1) (end 105.1 103.3) (width 0.2) (layer "B.Cu") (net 1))
 (segment (start 82.95 88.15) (end 82.8 88.3) (width 0.2) (layer "F.Cu") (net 23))
 (segment (start 82.8 88.3) (end 78.9 88.3) (width 0.2) (layer "F.Cu") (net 23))
 (segment (start 84.95 88.15) (end 82.95 88.15) (width 0.2) (layer "F.Cu") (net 23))
 (segment (start 80.4 105.3) (end 78.9 105.3) (width 0.2) (layer "F.Cu") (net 7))
 (segment (start 108.25 90.15) (end 106.35 90.15) (width 0.2) (layer "F.Cu") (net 7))
 (segment (start 106.35 90.15) (end 106.3 90.2) (width 0.2) (layer "F.Cu") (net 7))
 (via (at 106.3 90.2) (size 0.6) (drill 0.3) (layers "F.Cu" "B.Cu") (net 7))
 (via (at 80.4 105.3) (size 0.6) (drill 0.3) (layers "F.Cu" "B.Cu") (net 7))
 (segment (start 87.5 102.1) (end 94.4 102.1) (width 0.2) (layer "B.Cu") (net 7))
 (segment (start 87.5 102.1) (end 84.3 105.3) (width 0.2) (layer "B.Cu") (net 7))
 (segment (start 106.3 90.2) (end 94.4 102.1) (width 0.2) (layer "B.Cu") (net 7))
 (segment (start 84.3 105.3) (end 80.4 105.3) (width 0.2) (layer "B.Cu") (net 7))
 (segment (start 105.6 81.5) (end 105.6 83.4) (width 0.2) (layer "F.Cu") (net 11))
 (segment (start 80.4 99.3) (end 78.9 99.3) (width 0.2) (layer "F.Cu") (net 11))
 (via (at 80.4 99.3) (size 0.6) (drill 0.3) (layers "F.Cu" "B.Cu") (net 11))
 (via (at 105.6 83.4) (size 0.6) (drill 0.3) (layers "F.Cu" "B.Cu") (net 11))
 (segment (start 86.7 97.4) (end 84.8 99.3) (width 0.2) (layer "B.Cu") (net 11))
 (segment (start 86.7 97.4) (end 91.6 97.4) (width 0.2) (layer "B.Cu") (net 11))
 (segment (start 84.8 99.3) (end 80.4 99.3) (width 0.2) (layer "B.Cu") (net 11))
 (segment (start 105.6 83.4) (end 91.6 97.4) (width 0.2) (layer "B.Cu") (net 11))
 (segment (start 82.5 102.3) (end 78.9 102.3) (width 0.2) (layer "F.Cu") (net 30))
 (segment (start 84.95 102.15) (end 82.65 102.15) (width 0.2) (layer "F.Cu") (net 30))
 (segment (start 82.65 102.15) (end 82.5 102.3) (width 0.2) (layer "F.Cu") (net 30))
 (segment (start 108.25 84.15) (end 106.35 84.15) (width 0.2) (layer "F.Cu") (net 10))
 (segment (start 106.35 84.15) (end 106.3 84.2) (width 0.2) (layer "F.Cu") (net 10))
 (segment (start 80.4 101.3) (end 78.9 101.3) (width 0.2) (layer "F.Cu") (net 10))
 (via (at 80.4 101.3) (size 0.6) (drill 0.3) (layers "F.Cu" "B.Cu") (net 10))
 (via (at 106.3 84.2) (size 0.6) (drill 0.3) (layers "F.Cu" "B.Cu") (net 10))
 (segment (start 87.2 98.4) (end 84.3 101.3) (width 0.2) (layer "B.Cu") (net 10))
 (segment (start 87.2 98.4) (end 92.1 98.4) (width 0.2) (layer "B.Cu") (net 10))
 (segment (start 106.3 84.2) (end 92.1 98.4) (width 0.2) (layer "B.Cu") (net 10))
 (segment (start 84.3 101.3) (end 80.4 101.3) (width 0.2) (layer "B.Cu") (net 10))
 (segment (start 80.4 106.3) (end 78.9 106.3) (width 0.2) (layer "F.Cu") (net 6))
 (segment (start 106.35 92.15) (end 106.3 92.2) (width 0.2) (layer "F.Cu") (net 6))
 (segment (start 108.25 92.15) (end 106.35 92.15) (width 0.2) (layer "F.Cu") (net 6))
 (via (at 80.4 106.3) (size 0.6) (drill 0.3) (layers "F.Cu" "B.Cu") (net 6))
 (via (at 106.3 92.2) (size 0.6) (drill 0.3) (layers "F.Cu" "B.Cu") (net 6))
 (segment (start 84.7 106.3) (end 80.4 106.3) (width 0.2) (layer "B.Cu") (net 6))
 (segment (start 87.8 103.2) (end 95.3 103.2) (width 0.2) (layer "B.Cu") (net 6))
 (segment (start 106.3 92.2) (end 95.3 103.2) (width 0.2) (layer "B.Cu") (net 6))
 (segment (start 87.8 103.2) (end 84.7 106.3) (width 0.2) (layer "B.Cu") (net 6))
 (segment (start 106.35 100.15) (end 106.3 100.2) (width 0.2) (layer "F.Cu") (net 2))
 (segment (start 108.25 100.15) (end 106.35 100.15) (width 0.2) (layer "F.Cu") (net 2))
 (segment (start 80.4 110.3) (end 78.9 110.3) (width 0.2) (layer "F.Cu") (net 2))
 (via (at 106.3 100.2) (size 0.6) (drill 0.3) (layers "F.Cu" "B.Cu") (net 2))
 (via (at 80.4 110.3) (size 0.6) (drill 0.3) (layers "F.Cu" "B.Cu") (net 2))
 (segment (start 99.4 107.1) (end 90 107.1) (width 0.2) (layer "B.Cu") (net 2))
 (segment (start 106.3 100.2) (end 99.4 107.1) (width 0.2) (layer "B.Cu") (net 2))
 (segment (start 86.8 110.3) (end 80.4 110.3) (width 0.2) (layer "B.Cu") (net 2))
 (segment (start 90 107.1) (end 86.8 110.3) (width 0.2) (layer "B.Cu") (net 2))
 (segment (start 80.4 89.3) (end 78.9 89.3) (width 0.2) (layer "F.Cu") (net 16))
 (segment (start 95.6 81.5) (end 95.6 83.5) (width 0.2) (layer "F.Cu") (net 16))
 (via (at 80.4 89.3) (size 0.6) (drill 0.3) (layers "F.Cu" "B.Cu") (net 16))
 (via (at 95.6 83.5) (size 0.6) (drill 0.3) (layers "F.Cu" "B.Cu") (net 16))
 (segment (start 80.4 89.3) (end 89.8 89.3) (width 0.2) (layer "B.Cu") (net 16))
 (segment (start 89.8 89.3) (end 95.6 83.5) (width 0.2) (layer "B.Cu") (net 16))
 (segment (start 101.6 81.5) (end 101.6 83.5) (width 0.2) (layer "F.Cu") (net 13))
 (segment (start 80.4 95.3) (end 78.9 95.3) (width 0.2) (layer "F.Cu") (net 13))
 (via (at 80.4 95.3) (size 0.6) (drill 0.3) (layers "F.Cu" "B.Cu") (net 13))
 (via (at 101.6 83.5) (size 0.6) (drill 0.3) (layers "F.Cu" "B.Cu") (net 13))
 (segment (start 89.8 95.3) (end 80.4 95.3) (width 0.2) (layer "B.Cu") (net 13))
 (segment (start 101.6 83.5) (end 89.8 95.3) (width 0.2) (layer "B.Cu") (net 13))
 (segment (start 89.6 81.5) (end 89.6 76.5) (width 0.2) (layer "F.Cu") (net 19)))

